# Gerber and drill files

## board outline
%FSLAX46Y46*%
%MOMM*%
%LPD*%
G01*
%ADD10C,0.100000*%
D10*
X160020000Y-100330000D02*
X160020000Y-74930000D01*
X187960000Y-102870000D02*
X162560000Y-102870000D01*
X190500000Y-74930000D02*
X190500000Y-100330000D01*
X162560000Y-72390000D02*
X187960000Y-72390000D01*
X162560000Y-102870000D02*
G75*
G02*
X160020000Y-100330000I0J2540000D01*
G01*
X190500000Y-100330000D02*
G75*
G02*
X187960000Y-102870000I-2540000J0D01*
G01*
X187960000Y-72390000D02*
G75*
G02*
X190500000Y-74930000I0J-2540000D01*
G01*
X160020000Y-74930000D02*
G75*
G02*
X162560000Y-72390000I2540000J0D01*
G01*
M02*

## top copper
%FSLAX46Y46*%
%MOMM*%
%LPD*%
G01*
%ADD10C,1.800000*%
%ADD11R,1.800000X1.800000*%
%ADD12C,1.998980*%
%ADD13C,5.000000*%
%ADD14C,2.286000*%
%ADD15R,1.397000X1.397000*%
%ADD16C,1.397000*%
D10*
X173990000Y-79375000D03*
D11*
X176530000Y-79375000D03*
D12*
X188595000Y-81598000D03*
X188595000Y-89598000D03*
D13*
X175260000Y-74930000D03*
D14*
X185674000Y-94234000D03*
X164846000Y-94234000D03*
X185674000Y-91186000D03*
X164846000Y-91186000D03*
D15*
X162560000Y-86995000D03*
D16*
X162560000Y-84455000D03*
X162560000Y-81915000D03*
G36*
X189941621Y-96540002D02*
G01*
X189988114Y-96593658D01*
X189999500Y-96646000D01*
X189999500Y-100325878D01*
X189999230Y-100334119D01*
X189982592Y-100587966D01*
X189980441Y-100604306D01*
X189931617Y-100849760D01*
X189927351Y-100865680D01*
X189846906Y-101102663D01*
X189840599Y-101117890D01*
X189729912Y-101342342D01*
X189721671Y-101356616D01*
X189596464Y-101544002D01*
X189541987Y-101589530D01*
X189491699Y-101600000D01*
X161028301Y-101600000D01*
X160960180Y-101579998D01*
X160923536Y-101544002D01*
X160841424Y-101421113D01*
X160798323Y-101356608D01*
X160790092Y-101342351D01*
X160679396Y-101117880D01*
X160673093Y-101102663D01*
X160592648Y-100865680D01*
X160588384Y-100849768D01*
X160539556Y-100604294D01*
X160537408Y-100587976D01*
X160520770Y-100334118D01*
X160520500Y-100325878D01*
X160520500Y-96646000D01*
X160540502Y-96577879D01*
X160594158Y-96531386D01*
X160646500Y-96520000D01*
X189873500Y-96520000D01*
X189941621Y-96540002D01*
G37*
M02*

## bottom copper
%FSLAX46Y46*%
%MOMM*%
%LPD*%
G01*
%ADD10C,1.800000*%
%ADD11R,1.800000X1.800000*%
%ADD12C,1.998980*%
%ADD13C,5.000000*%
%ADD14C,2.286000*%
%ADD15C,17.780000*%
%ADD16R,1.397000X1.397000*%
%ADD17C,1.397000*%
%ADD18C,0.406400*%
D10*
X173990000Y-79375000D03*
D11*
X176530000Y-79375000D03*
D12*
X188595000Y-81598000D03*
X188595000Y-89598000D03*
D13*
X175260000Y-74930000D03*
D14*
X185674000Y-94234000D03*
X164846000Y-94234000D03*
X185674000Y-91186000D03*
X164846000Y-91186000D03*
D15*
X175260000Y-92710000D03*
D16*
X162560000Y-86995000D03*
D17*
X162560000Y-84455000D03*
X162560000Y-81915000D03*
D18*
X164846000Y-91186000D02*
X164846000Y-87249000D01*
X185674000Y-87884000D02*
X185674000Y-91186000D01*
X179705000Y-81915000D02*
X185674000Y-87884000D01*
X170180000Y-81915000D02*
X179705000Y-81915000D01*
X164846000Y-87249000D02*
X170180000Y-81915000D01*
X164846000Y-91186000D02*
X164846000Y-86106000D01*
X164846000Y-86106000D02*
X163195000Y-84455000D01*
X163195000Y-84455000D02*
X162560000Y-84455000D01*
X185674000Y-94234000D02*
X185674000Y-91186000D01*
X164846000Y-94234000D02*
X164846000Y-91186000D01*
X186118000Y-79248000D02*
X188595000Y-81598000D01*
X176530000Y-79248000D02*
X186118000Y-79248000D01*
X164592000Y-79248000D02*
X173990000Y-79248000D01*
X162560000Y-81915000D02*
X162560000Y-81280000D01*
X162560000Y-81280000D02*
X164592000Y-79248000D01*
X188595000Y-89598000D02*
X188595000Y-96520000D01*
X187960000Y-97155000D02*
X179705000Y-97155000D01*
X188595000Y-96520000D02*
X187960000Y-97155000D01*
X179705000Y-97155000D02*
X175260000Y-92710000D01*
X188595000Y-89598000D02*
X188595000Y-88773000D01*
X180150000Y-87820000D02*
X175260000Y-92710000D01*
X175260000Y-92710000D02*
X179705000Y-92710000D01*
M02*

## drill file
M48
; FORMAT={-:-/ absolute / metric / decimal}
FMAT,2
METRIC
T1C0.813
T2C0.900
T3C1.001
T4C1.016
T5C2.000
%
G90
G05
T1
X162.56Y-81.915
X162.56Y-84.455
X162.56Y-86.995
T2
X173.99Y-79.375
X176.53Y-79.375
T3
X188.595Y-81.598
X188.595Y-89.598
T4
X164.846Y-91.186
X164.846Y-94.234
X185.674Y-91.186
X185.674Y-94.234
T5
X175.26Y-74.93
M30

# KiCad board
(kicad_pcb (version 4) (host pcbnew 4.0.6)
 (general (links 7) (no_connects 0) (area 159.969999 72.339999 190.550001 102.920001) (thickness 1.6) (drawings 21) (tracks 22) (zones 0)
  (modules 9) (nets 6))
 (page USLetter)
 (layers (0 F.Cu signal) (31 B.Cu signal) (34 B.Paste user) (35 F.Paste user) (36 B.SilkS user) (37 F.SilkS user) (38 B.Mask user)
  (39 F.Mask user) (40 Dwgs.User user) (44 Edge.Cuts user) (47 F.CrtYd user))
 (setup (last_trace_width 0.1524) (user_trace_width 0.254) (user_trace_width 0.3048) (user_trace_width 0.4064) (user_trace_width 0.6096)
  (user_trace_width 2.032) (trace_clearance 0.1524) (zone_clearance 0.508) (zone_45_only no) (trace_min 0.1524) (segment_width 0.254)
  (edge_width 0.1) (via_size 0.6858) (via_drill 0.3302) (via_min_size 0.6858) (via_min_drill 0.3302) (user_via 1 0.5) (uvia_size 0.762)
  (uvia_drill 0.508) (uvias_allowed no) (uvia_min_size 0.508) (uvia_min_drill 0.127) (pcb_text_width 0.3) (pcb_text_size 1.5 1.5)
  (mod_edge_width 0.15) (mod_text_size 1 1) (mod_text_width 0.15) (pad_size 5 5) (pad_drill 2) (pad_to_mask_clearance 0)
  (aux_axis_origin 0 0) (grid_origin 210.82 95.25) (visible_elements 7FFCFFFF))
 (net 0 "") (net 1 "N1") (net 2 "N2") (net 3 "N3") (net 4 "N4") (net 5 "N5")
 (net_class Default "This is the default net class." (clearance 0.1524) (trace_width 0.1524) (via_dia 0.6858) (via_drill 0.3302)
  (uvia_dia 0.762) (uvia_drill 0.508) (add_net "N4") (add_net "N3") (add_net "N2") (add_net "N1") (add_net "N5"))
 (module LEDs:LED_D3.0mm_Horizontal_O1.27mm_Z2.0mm (layer F.Cu) (at 173.99 79.375)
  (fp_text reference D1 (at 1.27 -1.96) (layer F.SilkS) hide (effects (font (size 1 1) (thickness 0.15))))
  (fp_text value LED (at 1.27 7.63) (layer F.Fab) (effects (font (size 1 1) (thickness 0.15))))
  (pad 2 thru_hole circle (at 0 0) (size 1.8 1.8) (drill 0.9) (layers *.Cu *.Mask) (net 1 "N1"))
  (pad 1 thru_hole rect (at 2.54 0) (size 1.8 1.8) (drill 0.9) (layers *.Cu *.Mask) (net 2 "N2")))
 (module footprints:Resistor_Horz (layer F.Cu) (at 188.595 85.598 270)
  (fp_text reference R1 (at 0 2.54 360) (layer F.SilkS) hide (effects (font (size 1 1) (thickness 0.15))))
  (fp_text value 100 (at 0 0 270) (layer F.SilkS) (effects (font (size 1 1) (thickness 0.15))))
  (pad 1 thru_hole circle (at -4 0 270) (size 1.99898 1.99898) (drill 1.00076) (layers *.Cu *.SilkS *.Mask) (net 2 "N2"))
  (pad 2 thru_hole circle (at 4 0 270) (size 1.99898 1.99898) (drill 1.00076) (layers *.Cu *.SilkS *.Mask) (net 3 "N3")))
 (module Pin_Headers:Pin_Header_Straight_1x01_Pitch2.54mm (layer F.Cu) (at 175.26 74.93)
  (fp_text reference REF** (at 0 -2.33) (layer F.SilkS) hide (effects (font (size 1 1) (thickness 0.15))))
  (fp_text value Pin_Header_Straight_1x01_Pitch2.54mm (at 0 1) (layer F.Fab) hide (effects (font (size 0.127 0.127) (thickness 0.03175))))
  (pad 1 thru_hole circle (at 0 0) (size 5 5) (drill 2) (layers *.Cu *.Mask)))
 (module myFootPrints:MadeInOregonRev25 (layer F.Cu) (at 167.64 76.454)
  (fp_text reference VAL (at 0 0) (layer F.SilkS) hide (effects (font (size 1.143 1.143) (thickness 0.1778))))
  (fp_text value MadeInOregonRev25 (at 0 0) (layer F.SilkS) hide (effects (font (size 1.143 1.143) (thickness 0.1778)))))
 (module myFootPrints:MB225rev (layer F.Cu) (at 184.15 76.2)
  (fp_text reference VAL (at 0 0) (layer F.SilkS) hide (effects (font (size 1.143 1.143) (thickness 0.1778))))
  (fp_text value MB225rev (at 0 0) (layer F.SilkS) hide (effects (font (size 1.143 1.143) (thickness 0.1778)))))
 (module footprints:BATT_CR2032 (layer B.Cu) (at 175.26 92.71 180)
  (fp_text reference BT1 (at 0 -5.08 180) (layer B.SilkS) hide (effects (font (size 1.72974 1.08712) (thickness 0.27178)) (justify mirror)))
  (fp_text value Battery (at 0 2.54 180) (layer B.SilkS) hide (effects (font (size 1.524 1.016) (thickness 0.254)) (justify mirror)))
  (pad 1 thru_hole circle (at -10.414 -1.524 180) (size 2.286 2.286) (drill 1.016) (layers *.Cu *.Mask B.SilkS) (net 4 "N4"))
  (pad 1 thru_hole circle (at 10.414 -1.524 180) (size 2.286 2.286) (drill 1.016) (layers *.Cu *.Mask B.SilkS) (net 4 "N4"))
  (pad 1 thru_hole circle (at -10.414 1.524 180) (size 2.286 2.286) (drill 1.016) (layers *.Cu *.Mask B.SilkS) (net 4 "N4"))
  (pad 1 thru_hole circle (at 10.414 1.524 180) (size 2.286 2.286) (drill 1.016) (layers *.Cu *.Mask B.SilkS) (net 4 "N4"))
  (pad 2 smd circle (at 0 0 180) (size 17.78 17.78) (layers B.Cu B.Paste B.Mask) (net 3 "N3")))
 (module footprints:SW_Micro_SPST (layer F.Cu) (at 162.56 84.455 90)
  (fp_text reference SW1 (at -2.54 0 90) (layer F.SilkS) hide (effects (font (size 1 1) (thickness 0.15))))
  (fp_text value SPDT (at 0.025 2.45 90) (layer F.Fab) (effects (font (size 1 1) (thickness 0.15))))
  (pad 1 thru_hole rect (at -2.54 0 90) (size 1.397 1.397) (drill 0.8128) (layers *.Cu *.Mask F.SilkS) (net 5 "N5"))
  (pad 2 thru_hole circle (at 0 0 90) (size 1.397 1.397) (drill 0.8128) (layers *.Cu *.Mask F.SilkS) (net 4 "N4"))
  (pad 3 thru_hole circle (at 2.54 0 90) (size 1.397 1.397) (drill 0.8128) (layers *.Cu *.Mask F.SilkS) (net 1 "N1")))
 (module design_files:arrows (layer F.Cu) (at 177.546 81.788)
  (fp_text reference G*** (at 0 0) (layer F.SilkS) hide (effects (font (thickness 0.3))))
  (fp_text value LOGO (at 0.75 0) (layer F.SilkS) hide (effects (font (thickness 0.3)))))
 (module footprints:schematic (layer F.Cu) (at 175.26 87.503)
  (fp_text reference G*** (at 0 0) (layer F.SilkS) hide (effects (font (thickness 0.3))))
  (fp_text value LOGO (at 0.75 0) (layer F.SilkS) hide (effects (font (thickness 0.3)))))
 (gr_line (start 160.02 100.33) (end 160.02 74.93) (angle 90) (layer Edge.Cuts) (width 0.1))
 (gr_line (start 187.96 102.87) (end 162.56 102.87) (angle 90) (layer Edge.Cuts) (width 0.1))
 (gr_line (start 190.5 74.93) (end 190.5 100.33) (angle 90) (layer Edge.Cuts) (width 0.1))
 (gr_line (start 162.56 72.39) (end 187.96 72.39) (angle 90) (layer Edge.Cuts) (width 0.1))
 (gr_arc (start 162.56 100.33) (end 162.56 102.87) (angle 90) (layer Edge.Cuts) (width 0.1))
 (gr_arc (start 187.96 100.33) (end 190.5 100.33) (angle 90) (layer Edge.Cuts) (width 0.1))
 (gr_arc (start 187.96 74.93) (end 187.96 72.39) (angle 90) (layer Edge.Cuts) (width 0.1))
 (gr_arc (start 162.56 74.93) (end 160.02 74.93) (angle 90) (layer Edge.Cuts) (width 0.1))
 (segment (start 164.846 91.186) (end 164.846 87.249) (width 0.4064) (layer B.Cu) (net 4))
 (segment (start 185.674 87.884) (end 185.674 91.186) (width 0.4064) (layer B.Cu) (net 4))
 (segment (start 179.705 81.915) (end 185.674 87.884) (width 0.4064) (layer B.Cu) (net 4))
 (segment (start 170.18 81.915) (end 179.705 81.915) (width 0.4064) (layer B.Cu) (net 4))
 (segment (start 164.846 87.249) (end 170.18 81.915) (width 0.4064) (layer B.Cu) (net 4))
 (segment (start 164.846 91.186) (end 164.846 86.106) (width 0.4064) (layer B.Cu) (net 4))
 (segment (start 164.846 86.106) (end 163.195 84.455) (width 0.4064) (layer B.Cu) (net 4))
 (segment (start 163.195 84.455) (end 162.56 84.455) (width 0.4064) (layer B.Cu) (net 4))
 (segment (start 185.674 94.234) (end 185.674 91.186) (width 0.4064) (layer B.Cu) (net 4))
 (segment (start 164.846 94.234) (end 164.846 91.186) (width 0.4064) (layer B.Cu) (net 4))
 (segment (start 186.118 79.248) (end 188.595 81.598) (width 0.4064) (layer B.Cu) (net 2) (status 20))
 (segment (start 176.53 79.248) (end 186.118 79.248) (width 0.4064) (layer B.Cu) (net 2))
 (segment (start 164.592 79.248) (end 173.99 79.248) (width 0.4064) (layer B.Cu) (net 1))
 (segment (start 162.56 81.915) (end 162.56 81.28) (width 0.4064) (layer B.Cu) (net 1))
 (segment (start 162.56 81.28) (end 164.592 79.248) (width 0.4064) (layer B.Cu) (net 1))
 (segment (start 188.595 89.598) (end 188.595 96.52) (width 0.4064) (layer B.Cu) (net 3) (status 10))
 (segment (start 187.96 97.155) (end 179.705 97.155) (width 0.4064) (layer B.Cu) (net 3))
 (segment (start 188.595 96.52) (end 187.96 97.155) (width 0.4064) (layer B.Cu) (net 3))
 (segment (start 179.705 97.155) (end 175.26 92.71) (width 0.4064) (layer B.Cu) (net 3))
 (segment (start 188.595 89.598) (end 188.595 88.773) (width 0.4064) (layer B.Cu) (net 3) (status 30))
 (segment (start 180.15 87.82) (end 175.26 92.71) (width 0.4064) (layer B.Cu) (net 3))
 (segment (start 175.26 92.71) (end 179.705 92.71) (width 0.4064) (layer B.Cu) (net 3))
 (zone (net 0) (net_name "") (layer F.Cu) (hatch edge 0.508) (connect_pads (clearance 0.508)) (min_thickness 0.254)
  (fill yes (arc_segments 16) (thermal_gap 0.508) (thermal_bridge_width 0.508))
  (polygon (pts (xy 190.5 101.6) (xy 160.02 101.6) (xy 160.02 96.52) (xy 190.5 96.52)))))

